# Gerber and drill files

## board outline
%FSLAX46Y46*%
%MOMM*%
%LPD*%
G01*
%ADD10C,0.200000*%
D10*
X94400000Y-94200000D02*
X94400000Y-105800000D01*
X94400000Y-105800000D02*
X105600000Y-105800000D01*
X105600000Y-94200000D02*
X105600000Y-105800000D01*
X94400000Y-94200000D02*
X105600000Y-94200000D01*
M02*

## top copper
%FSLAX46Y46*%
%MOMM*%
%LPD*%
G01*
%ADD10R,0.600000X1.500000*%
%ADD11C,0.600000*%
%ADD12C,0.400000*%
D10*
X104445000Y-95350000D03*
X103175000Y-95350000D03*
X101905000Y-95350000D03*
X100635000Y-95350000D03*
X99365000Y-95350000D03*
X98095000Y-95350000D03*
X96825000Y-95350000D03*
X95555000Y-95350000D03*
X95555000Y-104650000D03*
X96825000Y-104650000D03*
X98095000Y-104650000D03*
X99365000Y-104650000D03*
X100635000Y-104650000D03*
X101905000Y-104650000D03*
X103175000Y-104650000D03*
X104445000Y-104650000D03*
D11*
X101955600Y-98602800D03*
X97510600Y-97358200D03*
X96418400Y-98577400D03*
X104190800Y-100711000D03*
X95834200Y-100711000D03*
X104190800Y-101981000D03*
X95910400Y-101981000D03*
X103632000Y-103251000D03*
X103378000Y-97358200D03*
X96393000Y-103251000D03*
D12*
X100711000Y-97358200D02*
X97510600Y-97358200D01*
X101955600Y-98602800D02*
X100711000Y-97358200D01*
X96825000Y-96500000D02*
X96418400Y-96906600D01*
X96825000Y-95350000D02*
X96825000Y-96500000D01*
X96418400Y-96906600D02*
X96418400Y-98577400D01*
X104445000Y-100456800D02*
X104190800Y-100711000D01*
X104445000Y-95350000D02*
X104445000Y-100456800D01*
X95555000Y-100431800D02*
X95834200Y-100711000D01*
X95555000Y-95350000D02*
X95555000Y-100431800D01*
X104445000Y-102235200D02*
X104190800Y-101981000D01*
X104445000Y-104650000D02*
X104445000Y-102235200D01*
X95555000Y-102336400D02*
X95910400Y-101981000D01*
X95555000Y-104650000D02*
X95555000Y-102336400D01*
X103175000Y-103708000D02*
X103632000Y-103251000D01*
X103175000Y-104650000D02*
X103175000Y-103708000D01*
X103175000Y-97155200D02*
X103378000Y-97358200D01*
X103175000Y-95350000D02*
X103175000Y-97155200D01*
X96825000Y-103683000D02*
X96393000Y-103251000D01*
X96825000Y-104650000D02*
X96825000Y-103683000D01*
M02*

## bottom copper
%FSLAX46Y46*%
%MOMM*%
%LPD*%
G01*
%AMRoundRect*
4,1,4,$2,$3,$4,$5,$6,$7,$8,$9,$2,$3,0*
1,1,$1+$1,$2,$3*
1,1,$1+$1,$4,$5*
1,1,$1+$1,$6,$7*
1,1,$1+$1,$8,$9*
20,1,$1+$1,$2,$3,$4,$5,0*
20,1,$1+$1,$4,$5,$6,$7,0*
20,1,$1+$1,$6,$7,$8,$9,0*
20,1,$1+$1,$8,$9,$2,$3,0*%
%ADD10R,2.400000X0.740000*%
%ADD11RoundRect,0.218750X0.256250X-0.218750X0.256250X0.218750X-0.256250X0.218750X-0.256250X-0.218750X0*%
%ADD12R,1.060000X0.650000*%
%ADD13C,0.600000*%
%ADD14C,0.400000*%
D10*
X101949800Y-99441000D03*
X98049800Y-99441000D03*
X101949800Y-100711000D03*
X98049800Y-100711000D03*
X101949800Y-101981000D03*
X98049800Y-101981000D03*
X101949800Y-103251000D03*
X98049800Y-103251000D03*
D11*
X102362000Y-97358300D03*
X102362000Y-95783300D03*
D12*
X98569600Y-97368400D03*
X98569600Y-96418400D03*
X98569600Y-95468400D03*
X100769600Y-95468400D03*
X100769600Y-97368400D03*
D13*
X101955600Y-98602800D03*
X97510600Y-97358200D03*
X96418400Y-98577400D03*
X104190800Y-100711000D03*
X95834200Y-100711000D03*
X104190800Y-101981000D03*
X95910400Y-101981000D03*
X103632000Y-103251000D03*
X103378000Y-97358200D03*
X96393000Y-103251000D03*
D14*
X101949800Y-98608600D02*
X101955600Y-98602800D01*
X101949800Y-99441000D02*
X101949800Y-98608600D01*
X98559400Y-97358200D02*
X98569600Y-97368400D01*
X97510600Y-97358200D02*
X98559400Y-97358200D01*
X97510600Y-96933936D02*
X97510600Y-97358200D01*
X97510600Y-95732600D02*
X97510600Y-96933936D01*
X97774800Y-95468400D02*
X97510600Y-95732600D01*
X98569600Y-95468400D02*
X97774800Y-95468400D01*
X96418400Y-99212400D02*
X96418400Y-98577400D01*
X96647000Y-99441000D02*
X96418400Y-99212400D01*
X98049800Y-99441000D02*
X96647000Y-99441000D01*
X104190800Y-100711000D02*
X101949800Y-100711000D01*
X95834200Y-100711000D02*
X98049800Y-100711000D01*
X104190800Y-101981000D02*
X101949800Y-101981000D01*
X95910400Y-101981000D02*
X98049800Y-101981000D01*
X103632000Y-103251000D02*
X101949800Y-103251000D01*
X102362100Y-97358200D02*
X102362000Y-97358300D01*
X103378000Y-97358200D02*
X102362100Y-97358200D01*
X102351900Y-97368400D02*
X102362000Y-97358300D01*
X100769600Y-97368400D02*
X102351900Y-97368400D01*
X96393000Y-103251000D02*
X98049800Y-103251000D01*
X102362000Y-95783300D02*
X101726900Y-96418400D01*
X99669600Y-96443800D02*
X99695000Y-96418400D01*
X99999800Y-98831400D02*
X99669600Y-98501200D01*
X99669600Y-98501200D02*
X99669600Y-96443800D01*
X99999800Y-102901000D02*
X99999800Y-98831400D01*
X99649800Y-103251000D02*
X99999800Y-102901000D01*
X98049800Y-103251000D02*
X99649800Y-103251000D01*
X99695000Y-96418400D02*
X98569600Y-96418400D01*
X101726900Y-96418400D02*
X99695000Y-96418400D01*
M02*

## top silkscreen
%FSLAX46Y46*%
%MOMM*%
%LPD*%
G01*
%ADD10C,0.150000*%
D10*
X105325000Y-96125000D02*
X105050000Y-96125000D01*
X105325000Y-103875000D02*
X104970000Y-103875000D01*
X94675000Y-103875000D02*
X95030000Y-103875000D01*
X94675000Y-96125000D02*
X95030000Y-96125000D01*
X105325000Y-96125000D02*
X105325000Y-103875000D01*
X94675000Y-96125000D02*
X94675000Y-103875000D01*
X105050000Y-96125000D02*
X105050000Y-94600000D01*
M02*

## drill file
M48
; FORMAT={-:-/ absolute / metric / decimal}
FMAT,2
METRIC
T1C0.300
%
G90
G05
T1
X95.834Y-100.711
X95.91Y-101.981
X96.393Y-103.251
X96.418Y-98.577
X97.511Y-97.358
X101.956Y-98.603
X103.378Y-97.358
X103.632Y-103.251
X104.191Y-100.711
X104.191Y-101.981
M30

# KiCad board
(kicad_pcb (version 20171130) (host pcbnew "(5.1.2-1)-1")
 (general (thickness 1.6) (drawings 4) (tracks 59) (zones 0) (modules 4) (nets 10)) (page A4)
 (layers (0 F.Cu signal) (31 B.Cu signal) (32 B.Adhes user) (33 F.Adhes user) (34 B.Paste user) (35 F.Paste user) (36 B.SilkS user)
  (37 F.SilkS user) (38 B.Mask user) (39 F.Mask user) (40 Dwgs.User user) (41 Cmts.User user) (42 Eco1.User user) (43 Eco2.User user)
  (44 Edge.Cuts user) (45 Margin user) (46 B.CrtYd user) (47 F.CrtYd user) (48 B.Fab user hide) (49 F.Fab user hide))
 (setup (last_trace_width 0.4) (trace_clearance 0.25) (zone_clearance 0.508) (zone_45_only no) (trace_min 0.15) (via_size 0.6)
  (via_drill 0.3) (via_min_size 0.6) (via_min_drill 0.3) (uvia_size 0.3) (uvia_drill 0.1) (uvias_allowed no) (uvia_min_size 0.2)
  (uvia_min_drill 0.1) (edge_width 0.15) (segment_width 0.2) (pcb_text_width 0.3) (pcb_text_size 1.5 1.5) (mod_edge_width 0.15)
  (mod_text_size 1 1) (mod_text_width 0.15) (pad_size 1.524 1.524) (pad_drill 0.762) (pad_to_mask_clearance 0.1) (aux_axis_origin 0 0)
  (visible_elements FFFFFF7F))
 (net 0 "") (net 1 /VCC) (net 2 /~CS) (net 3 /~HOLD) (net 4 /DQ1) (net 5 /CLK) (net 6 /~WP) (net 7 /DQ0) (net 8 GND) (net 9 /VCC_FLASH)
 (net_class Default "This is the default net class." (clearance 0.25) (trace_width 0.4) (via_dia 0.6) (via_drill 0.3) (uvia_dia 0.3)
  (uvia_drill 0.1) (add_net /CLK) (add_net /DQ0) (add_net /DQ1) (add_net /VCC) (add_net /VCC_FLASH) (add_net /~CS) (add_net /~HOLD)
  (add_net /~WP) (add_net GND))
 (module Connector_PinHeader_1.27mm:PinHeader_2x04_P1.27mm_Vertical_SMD (layer B.Cu) (at 99.9998 101.346 180)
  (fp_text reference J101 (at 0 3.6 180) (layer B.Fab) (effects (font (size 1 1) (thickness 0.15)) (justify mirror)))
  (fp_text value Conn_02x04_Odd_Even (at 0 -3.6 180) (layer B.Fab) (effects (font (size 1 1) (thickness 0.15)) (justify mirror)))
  (pad 1 smd rect (at -1.95 1.905 180) (size 2.4 0.74) (layers B.Cu B.Paste B.Mask) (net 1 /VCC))
  (pad 2 smd rect (at 1.95 1.905 180) (size 2.4 0.74) (layers B.Cu B.Paste B.Mask) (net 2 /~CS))
  (pad 3 smd rect (at -1.95 0.635 180) (size 2.4 0.74) (layers B.Cu B.Paste B.Mask) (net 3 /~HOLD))
  (pad 4 smd rect (at 1.95 0.635 180) (size 2.4 0.74) (layers B.Cu B.Paste B.Mask) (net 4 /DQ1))
  (pad 5 smd rect (at -1.95 -0.635 180) (size 2.4 0.74) (layers B.Cu B.Paste B.Mask) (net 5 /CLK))
  (pad 6 smd rect (at 1.95 -0.635 180) (size 2.4 0.74) (layers B.Cu B.Paste B.Mask) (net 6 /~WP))
  (pad 7 smd rect (at -1.95 -1.905 180) (size 2.4 0.74) (layers B.Cu B.Paste B.Mask) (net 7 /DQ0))
  (pad 8 smd rect (at 1.95 -1.905 180) (size 2.4 0.74) (layers B.Cu B.Paste B.Mask) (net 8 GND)))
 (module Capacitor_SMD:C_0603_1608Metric (layer B.Cu) (at 102.362 96.5708 90)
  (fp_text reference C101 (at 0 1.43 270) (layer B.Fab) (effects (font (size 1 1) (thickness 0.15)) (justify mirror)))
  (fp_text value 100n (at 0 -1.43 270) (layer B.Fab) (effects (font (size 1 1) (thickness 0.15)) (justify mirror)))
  (pad 1 smd roundrect (at -0.7875 0 90) (size 0.875 0.95) (layers B.Cu B.Paste B.Mask) (roundrect_rratio 0.25) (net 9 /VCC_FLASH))
  (pad 2 smd roundrect (at 0.7875 0 90) (size 0.875 0.95) (layers B.Cu B.Paste B.Mask) (roundrect_rratio 0.25) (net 8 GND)))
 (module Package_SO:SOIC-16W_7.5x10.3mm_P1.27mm (layer F.Cu) (at 100 100 270)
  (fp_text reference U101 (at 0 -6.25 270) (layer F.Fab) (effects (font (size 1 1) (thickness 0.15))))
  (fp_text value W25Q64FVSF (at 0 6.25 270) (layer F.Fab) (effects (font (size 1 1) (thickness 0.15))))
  (fp_line (start -3.875 -5.325) (end -3.875 -5.05) (layer F.SilkS) (width 0.15))
  (fp_line (start 3.875 -5.325) (end 3.875 -4.97) (layer F.SilkS) (width 0.15))
  (fp_line (start 3.875 5.325) (end 3.875 4.97) (layer F.SilkS) (width 0.15))
  (fp_line (start -3.875 5.325) (end -3.875 4.97) (layer F.SilkS) (width 0.15))
  (fp_line (start -3.875 -5.325) (end 3.875 -5.325) (layer F.SilkS) (width 0.15))
  (fp_line (start -3.875 5.325) (end 3.875 5.325) (layer F.SilkS) (width 0.15))
  (fp_line (start -3.875 -5.05) (end -5.4 -5.05) (layer F.SilkS) (width 0.15))
  (pad 1 smd rect (at -4.65 -4.445 270) (size 1.5 0.6) (layers F.Cu F.Paste F.Mask) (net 3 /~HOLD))
  (pad 2 smd rect (at -4.65 -3.175 270) (size 1.5 0.6) (layers F.Cu F.Paste F.Mask) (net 9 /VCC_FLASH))
  (pad 3 smd rect (at -4.65 -1.905 270) (size 1.5 0.6) (layers F.Cu F.Paste F.Mask))
  (pad 4 smd rect (at -4.65 -0.635 270) (size 1.5 0.6) (layers F.Cu F.Paste F.Mask))
  (pad 5 smd rect (at -4.65 0.635 270) (size 1.5 0.6) (layers F.Cu F.Paste F.Mask))
  (pad 6 smd rect (at -4.65 1.905 270) (size 1.5 0.6) (layers F.Cu F.Paste F.Mask))
  (pad 7 smd rect (at -4.65 3.175 270) (size 1.5 0.6) (layers F.Cu F.Paste F.Mask) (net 2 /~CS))
  (pad 8 smd rect (at -4.65 4.445 270) (size 1.5 0.6) (layers F.Cu F.Paste F.Mask) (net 4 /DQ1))
  (pad 9 smd rect (at 4.65 4.445 270) (size 1.5 0.6) (layers F.Cu F.Paste F.Mask) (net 6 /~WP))
  (pad 10 smd rect (at 4.65 3.175 270) (size 1.5 0.6) (layers F.Cu F.Paste F.Mask) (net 8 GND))
  (pad 11 smd rect (at 4.65 1.905 270) (size 1.5 0.6) (layers F.Cu F.Paste F.Mask))
  (pad 12 smd rect (at 4.65 0.635 270) (size 1.5 0.6) (layers F.Cu F.Paste F.Mask))
  (pad 13 smd rect (at 4.65 -0.635 270) (size 1.5 0.6) (layers F.Cu F.Paste F.Mask))
  (pad 14 smd rect (at 4.65 -1.905 270) (size 1.5 0.6) (layers F.Cu F.Paste F.Mask))
  (pad 15 smd rect (at 4.65 -3.175 270) (size 1.5 0.6) (layers F.Cu F.Paste F.Mask) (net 7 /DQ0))
  (pad 16 smd rect (at 4.65 -4.445 270) (size 1.5 0.6) (layers F.Cu F.Paste F.Mask) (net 5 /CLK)))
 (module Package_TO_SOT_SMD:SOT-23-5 (layer B.Cu) (at 99.6696 96.4184)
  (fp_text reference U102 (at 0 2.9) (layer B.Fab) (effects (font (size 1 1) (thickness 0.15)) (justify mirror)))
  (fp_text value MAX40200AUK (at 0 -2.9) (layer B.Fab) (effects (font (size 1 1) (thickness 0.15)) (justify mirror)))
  (pad 1 smd rect (at -1.1 0.95) (size 1.06 0.65) (layers B.Cu B.Paste B.Mask) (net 1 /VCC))
  (pad 2 smd rect (at -1.1 0) (size 1.06 0.65) (layers B.Cu B.Paste B.Mask) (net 8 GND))
  (pad 3 smd rect (at -1.1 -0.95) (size 1.06 0.65) (layers B.Cu B.Paste B.Mask) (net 1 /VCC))
  (pad 4 smd rect (at 1.1 -0.95) (size 1.06 0.65) (layers B.Cu B.Paste B.Mask))
  (pad 5 smd rect (at 1.1 0.95) (size 1.06 0.65) (layers B.Cu B.Paste B.Mask) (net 9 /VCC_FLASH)))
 (gr_line (start 94.4 94.2) (end 94.4 105.8) (layer Edge.Cuts) (width 0.2))
 (gr_line (start 94.4 105.8) (end 105.6 105.8) (layer Edge.Cuts) (width 0.2))
 (gr_line (start 105.6 94.2) (end 105.6 105.8) (layer Edge.Cuts) (width 0.2))
 (gr_line (start 94.4 94.2) (end 105.6 94.2) (layer Edge.Cuts) (width 0.2))
 (via (at 101.9556 98.6028) (size 0.6) (drill 0.3) (layers F.Cu B.Cu) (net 1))
 (segment (start 101.9498 98.6086) (end 101.9556 98.6028) (width 0.4) (layer B.Cu) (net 1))
 (segment (start 101.9498 99.441) (end 101.9498 98.6086) (width 0.4) (layer B.Cu) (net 1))
 (via (at 97.5106 97.3582) (size 0.6) (drill 0.3) (layers F.Cu B.Cu) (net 1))
 (segment (start 100.711 97.3582) (end 97.5106 97.3582) (width 0.4) (layer F.Cu) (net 1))
 (segment (start 101.9556 98.6028) (end 100.711 97.3582) (width 0.4) (layer F.Cu) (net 1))
 (segment (start 98.5594 97.3582) (end 98.5696 97.3684) (width 0.4) (layer B.Cu) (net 1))
 (segment (start 97.5106 97.3582) (end 98.5594 97.3582) (width 0.4) (layer B.Cu) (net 1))
 (segment (start 97.5106 96.933936) (end 97.5106 97.3582) (width 0.4) (layer B.Cu) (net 1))
 (segment (start 97.5106 95.7326) (end 97.5106 96.933936) (width 0.4) (layer B.Cu) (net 1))
 (segment (start 97.7748 95.4684) (end 97.5106 95.7326) (width 0.4) (layer B.Cu) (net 1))
 (segment (start 98.5696 95.4684) (end 97.7748 95.4684) (width 0.4) (layer B.Cu) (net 1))
 (segment (start 96.825 96.5) (end 96.4184 96.9066) (width 0.4) (layer F.Cu) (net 2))
 (segment (start 96.825 95.35) (end 96.825 96.5) (width 0.4) (layer F.Cu) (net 2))
 (via (at 96.4184 98.5774) (size 0.6) (drill 0.3) (layers F.Cu B.Cu) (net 2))
 (segment (start 96.4184 96.9066) (end 96.4184 98.5774) (width 0.4) (layer F.Cu) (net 2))
 (segment (start 96.4184 99.2124) (end 96.4184 98.5774) (width 0.4) (layer B.Cu) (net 2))
 (segment (start 96.647 99.441) (end 96.4184 99.2124) (width 0.4) (layer B.Cu) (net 2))
 (segment (start 98.0498 99.441) (end 96.647 99.441) (width 0.4) (layer B.Cu) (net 2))
 (via (at 104.1908 100.711) (size 0.6) (drill 0.3) (layers F.Cu B.Cu) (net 3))
 (segment (start 104.445 100.4568) (end 104.1908 100.711) (width 0.4) (layer F.Cu) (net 3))
 (segment (start 104.445 95.35) (end 104.445 100.4568) (width 0.4) (layer F.Cu) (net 3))
 (segment (start 104.1908 100.711) (end 101.9498 100.711) (width 0.4) (layer B.Cu) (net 3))
 (via (at 95.8342 100.711) (size 0.6) (drill 0.3) (layers F.Cu B.Cu) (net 4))
 (segment (start 95.555 100.4318) (end 95.8342 100.711) (width 0.4) (layer F.Cu) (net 4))
 (segment (start 95.555 95.35) (end 95.555 100.4318) (width 0.4) (layer F.Cu) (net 4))
 (segment (start 95.8342 100.711) (end 98.0498 100.711) (width 0.4) (layer B.Cu) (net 4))
 (via (at 104.1908 101.981) (size 0.6) (drill 0.3) (layers F.Cu B.Cu) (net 5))
 (segment (start 104.445 102.2352) (end 104.1908 101.981) (width 0.4) (layer F.Cu) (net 5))
 (segment (start 104.445 104.65) (end 104.445 102.2352) (width 0.4) (layer F.Cu) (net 5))
 (segment (start 104.1908 101.981) (end 101.9498 101.981) (width 0.4) (layer B.Cu) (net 5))
 (via (at 95.9104 101.981) (size 0.6) (drill 0.3) (layers F.Cu B.Cu) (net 6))
 (segment (start 95.555 102.3364) (end 95.9104 101.981) (width 0.4) (layer F.Cu) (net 6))
 (segment (start 95.555 104.65) (end 95.555 102.3364) (width 0.4) (layer F.Cu) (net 6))
 (segment (start 95.9104 101.981) (end 98.0498 101.981) (width 0.4) (layer B.Cu) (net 6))
 (via (at 103.632 103.251) (size 0.6) (drill 0.3) (layers F.Cu B.Cu) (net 7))
 (segment (start 103.175 103.708) (end 103.632 103.251) (width 0.4) (layer F.Cu) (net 7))
 (segment (start 103.175 104.65) (end 103.175 103.708) (width 0.4) (layer F.Cu) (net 7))
 (segment (start 103.632 103.251) (end 101.9498 103.251) (width 0.4) (layer B.Cu) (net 7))
 (via (at 103.378 97.3582) (size 0.6) (drill 0.3) (layers F.Cu B.Cu) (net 9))
 (segment (start 103.175 97.1552) (end 103.378 97.3582) (width 0.4) (layer F.Cu) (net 9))
 (segment (start 103.175 95.35) (end 103.175 97.1552) (width 0.4) (layer F.Cu) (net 9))
 (segment (start 102.3621 97.3582) (end 102.362 97.3583) (width 0.4) (layer B.Cu) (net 9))
 (segment (start 103.378 97.3582) (end 102.3621 97.3582) (width 0.4) (layer B.Cu) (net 9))
 (segment (start 102.3519 97.3684) (end 102.362 97.3583) (width 0.4) (layer B.Cu) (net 9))
 (segment (start 100.7696 97.3684) (end 102.3519 97.3684) (width 0.4) (layer B.Cu) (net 9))
 (via (at 96.393 103.251) (size 0.6) (drill 0.3) (layers F.Cu B.Cu) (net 8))
 (segment (start 96.825 103.683) (end 96.393 103.251) (width 0.4) (layer F.Cu) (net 8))
 (segment (start 96.825 104.65) (end 96.825 103.683) (width 0.4) (layer F.Cu) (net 8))
 (segment (start 96.393 103.251) (end 98.0498 103.251) (width 0.4) (layer B.Cu) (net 8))
 (segment (start 102.362 95.7833) (end 101.7269 96.4184) (width 0.4) (layer B.Cu) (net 8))
 (segment (start 99.6696 96.4438) (end 99.695 96.4184) (width 0.4) (layer B.Cu) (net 8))
 (segment (start 99.9998 98.8314) (end 99.6696 98.5012) (width 0.4) (layer B.Cu) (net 8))
 (segment (start 99.6696 98.5012) (end 99.6696 96.4438) (width 0.4) (layer B.Cu) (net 8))
 (segment (start 99.9998 102.901) (end 99.9998 98.8314) (width 0.4) (layer B.Cu) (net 8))
 (segment (start 99.6498 103.251) (end 99.9998 102.901) (width 0.4) (layer B.Cu) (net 8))
 (segment (start 98.0498 103.251) (end 99.6498 103.251) (width 0.4) (layer B.Cu) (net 8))
 (segment (start 99.695 96.4184) (end 98.5696 96.4184) (width 0.4) (layer B.Cu) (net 8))
 (segment (start 101.7269 96.4184) (end 99.695 96.4184) (width 0.4) (layer B.Cu) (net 8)))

